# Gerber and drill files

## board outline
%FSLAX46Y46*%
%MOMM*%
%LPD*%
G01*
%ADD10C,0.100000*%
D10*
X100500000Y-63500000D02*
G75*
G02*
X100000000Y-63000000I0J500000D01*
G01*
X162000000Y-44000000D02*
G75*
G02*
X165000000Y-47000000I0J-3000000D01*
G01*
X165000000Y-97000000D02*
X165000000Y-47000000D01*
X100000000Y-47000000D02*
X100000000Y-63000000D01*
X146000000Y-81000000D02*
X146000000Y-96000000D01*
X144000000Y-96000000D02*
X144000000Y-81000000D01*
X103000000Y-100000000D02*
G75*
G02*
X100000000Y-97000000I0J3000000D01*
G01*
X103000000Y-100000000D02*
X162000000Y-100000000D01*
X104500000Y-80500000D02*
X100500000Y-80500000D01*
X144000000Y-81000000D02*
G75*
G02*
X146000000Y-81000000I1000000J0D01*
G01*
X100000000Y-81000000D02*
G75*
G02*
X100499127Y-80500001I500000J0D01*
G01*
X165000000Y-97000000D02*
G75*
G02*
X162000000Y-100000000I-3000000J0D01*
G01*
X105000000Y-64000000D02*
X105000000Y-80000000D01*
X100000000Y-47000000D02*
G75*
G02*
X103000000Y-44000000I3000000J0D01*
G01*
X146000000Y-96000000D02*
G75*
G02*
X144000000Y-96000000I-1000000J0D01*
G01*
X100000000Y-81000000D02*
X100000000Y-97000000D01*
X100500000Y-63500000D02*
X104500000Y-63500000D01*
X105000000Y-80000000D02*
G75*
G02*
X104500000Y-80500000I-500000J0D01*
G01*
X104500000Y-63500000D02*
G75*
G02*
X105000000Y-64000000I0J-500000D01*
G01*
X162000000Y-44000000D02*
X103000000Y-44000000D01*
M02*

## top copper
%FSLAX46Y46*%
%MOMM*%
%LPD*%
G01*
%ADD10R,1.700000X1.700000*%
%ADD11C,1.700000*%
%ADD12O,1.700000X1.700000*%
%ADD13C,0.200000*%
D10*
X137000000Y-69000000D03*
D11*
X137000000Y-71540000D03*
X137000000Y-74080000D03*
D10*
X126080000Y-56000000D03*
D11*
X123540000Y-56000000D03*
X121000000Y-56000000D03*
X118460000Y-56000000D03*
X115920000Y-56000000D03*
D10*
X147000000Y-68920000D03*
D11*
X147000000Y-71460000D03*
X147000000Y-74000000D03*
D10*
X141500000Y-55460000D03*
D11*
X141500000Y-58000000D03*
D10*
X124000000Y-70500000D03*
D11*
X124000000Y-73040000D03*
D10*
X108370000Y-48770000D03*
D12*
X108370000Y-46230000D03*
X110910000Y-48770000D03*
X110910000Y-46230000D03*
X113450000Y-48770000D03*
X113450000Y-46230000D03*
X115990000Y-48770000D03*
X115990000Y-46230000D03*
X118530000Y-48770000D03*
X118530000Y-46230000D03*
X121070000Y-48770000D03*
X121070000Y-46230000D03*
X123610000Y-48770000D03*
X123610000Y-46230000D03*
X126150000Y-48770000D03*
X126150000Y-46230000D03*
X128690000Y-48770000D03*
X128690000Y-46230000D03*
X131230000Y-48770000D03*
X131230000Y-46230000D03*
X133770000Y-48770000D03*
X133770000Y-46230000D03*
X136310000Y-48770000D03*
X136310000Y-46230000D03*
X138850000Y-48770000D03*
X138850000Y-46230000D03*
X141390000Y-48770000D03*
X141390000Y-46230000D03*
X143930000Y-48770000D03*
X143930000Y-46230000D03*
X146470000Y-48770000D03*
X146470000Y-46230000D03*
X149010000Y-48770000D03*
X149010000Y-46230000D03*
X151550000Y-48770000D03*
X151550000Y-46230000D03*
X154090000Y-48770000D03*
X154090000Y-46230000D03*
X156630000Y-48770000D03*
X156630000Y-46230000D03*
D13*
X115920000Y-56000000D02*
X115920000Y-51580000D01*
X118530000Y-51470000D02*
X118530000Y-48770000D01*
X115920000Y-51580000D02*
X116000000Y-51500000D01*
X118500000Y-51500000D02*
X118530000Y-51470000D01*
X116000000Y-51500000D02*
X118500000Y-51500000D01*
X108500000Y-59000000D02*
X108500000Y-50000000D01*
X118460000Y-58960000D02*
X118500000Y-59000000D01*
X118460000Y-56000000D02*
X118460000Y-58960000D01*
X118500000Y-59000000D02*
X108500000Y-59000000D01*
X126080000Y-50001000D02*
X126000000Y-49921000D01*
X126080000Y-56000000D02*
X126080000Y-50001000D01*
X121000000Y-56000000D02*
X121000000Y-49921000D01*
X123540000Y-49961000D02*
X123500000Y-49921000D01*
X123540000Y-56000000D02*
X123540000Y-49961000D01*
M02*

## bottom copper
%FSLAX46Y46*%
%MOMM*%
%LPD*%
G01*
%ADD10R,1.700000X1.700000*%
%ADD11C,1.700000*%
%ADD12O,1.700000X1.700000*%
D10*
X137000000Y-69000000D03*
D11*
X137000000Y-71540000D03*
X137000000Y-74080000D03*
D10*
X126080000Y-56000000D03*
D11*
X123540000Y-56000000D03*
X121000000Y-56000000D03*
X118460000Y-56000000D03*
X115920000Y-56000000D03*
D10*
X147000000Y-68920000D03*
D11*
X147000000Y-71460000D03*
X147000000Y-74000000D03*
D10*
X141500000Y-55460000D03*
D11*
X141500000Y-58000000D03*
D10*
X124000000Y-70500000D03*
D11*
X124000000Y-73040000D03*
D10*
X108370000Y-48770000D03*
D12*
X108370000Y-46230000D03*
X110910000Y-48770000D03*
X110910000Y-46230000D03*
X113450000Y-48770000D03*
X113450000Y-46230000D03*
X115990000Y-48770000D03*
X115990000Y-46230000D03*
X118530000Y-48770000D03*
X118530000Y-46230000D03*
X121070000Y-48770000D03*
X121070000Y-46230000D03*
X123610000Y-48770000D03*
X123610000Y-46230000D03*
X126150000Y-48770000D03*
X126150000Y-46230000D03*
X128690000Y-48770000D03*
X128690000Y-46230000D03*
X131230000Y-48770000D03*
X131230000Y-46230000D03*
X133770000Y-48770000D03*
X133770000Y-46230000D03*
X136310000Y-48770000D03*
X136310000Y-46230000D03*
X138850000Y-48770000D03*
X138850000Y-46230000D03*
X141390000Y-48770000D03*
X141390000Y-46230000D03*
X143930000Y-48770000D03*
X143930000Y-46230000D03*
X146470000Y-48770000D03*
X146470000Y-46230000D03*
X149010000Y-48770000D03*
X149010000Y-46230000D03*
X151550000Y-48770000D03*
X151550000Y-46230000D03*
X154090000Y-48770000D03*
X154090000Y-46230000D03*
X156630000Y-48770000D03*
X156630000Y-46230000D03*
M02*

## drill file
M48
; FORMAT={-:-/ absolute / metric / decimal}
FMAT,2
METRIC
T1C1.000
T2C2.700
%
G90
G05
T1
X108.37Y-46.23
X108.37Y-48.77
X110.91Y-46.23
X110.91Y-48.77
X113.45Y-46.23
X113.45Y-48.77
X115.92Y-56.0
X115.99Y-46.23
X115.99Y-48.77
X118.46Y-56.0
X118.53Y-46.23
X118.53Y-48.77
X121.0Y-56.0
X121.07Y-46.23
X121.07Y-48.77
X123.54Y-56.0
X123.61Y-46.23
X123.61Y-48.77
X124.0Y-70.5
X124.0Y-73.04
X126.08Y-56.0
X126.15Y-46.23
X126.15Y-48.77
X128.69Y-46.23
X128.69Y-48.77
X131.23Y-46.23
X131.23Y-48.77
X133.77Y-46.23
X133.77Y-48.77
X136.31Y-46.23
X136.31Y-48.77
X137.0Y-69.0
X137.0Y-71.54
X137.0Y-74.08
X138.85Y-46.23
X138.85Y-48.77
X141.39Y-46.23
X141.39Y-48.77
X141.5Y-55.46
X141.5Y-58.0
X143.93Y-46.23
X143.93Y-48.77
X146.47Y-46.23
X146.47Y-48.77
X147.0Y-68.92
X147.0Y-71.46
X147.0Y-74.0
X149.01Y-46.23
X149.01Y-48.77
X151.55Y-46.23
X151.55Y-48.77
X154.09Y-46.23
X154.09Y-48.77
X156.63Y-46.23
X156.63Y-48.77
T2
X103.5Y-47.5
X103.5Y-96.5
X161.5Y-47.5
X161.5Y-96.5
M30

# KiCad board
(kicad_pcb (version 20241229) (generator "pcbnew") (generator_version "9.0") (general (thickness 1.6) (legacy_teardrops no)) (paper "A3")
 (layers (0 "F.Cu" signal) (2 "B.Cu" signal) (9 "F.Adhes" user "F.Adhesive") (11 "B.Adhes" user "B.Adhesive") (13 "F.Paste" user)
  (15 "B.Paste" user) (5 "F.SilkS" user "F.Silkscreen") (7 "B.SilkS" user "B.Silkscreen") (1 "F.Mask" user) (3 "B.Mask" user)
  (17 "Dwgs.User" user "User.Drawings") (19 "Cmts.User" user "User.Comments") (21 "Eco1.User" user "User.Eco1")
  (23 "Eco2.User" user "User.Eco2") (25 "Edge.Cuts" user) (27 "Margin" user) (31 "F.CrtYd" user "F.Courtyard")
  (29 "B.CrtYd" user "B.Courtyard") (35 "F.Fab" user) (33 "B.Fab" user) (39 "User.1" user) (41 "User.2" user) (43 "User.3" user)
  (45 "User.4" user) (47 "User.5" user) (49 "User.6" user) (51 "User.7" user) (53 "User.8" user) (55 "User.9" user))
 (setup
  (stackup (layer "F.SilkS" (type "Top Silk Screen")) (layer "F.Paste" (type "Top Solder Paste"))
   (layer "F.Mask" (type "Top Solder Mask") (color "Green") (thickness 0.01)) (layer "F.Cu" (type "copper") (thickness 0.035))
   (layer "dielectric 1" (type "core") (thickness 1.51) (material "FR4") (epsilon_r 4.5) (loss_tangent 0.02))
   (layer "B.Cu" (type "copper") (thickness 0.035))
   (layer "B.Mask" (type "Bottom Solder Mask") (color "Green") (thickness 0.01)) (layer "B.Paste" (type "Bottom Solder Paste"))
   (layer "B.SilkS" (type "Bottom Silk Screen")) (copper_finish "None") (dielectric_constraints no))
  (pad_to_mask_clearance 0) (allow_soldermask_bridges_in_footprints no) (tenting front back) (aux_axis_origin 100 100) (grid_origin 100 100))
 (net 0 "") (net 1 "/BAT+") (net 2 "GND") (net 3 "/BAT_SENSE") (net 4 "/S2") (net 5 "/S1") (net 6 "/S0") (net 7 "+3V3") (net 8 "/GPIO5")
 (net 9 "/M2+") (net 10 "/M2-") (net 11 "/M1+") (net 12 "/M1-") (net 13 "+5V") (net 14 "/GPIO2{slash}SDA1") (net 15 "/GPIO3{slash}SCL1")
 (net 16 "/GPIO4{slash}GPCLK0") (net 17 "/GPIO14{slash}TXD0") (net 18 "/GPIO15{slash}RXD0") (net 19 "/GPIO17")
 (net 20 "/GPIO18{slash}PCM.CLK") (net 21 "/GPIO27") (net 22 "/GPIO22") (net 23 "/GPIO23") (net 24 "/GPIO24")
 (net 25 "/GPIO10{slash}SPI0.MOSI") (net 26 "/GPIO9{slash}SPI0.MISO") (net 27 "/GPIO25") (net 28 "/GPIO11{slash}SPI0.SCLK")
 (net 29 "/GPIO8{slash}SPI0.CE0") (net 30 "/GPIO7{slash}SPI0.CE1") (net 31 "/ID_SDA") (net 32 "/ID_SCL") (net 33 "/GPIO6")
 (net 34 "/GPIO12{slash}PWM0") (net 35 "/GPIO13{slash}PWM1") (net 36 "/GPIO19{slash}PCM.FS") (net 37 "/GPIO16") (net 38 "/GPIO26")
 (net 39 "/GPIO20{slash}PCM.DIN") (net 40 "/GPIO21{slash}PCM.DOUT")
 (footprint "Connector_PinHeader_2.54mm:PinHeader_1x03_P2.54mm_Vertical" (layer "F.Cu") (at 137 69)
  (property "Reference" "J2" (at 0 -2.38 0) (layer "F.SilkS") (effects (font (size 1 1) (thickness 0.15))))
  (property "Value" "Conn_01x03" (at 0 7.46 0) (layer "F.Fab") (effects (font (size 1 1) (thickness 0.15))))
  (pad "1" thru_hole rect (at 0 0) (size 1.7 1.7) (drill 1) (layers "*.Cu" "*.Mask") (remove_unused_layers no) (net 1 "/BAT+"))
  (pad "2" thru_hole circle (at 0 2.54) (size 1.7 1.7) (drill 1) (layers "*.Cu" "*.Mask") (remove_unused_layers no) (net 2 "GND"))
  (pad "3" thru_hole circle (at 0 5.08) (size 1.7 1.7) (drill 1) (layers "*.Cu" "*.Mask") (remove_unused_layers no) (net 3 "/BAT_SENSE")))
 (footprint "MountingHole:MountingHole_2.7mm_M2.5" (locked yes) (layer "F.Cu") (at 161.5 47.5)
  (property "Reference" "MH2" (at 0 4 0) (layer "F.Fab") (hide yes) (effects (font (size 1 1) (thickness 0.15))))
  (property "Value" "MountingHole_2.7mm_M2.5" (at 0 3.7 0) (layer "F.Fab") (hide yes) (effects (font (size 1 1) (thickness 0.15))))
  (pad "" np_thru_hole circle (at 0 0) (size 2.7 2.7) (drill 2.7) (layers "*.Cu" "*.Mask")))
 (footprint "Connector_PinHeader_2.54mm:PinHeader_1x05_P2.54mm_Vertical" (layer "F.Cu") (at 126.08 56 -90)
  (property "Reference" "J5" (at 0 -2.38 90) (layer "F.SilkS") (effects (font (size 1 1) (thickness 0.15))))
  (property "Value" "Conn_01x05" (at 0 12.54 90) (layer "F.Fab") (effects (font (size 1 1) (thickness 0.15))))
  (pad "1" thru_hole rect (at 0 0 270) (size 1.7 1.7) (drill 1) (layers "*.Cu" "*.Mask") (remove_unused_layers no) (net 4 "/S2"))
  (pad "2" thru_hole circle (at 0 2.54 270) (size 1.7 1.7) (drill 1) (layers "*.Cu" "*.Mask") (remove_unused_layers no) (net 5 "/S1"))
  (pad "3" thru_hole circle (at 0 5.08 270) (size 1.7 1.7) (drill 1) (layers "*.Cu" "*.Mask") (remove_unused_layers no) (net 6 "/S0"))
  (pad "4" thru_hole circle (at 0 7.62 270) (size 1.7 1.7) (drill 1) (layers "*.Cu" "*.Mask") (remove_unused_layers no) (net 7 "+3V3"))
  (pad "5" thru_hole circle (at 0 10.16 270) (size 1.7 1.7) (drill 1) (layers "*.Cu" "*.Mask") (remove_unused_layers no) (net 2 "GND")))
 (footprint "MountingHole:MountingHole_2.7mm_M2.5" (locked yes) (layer "F.Cu") (at 103.5 96.5)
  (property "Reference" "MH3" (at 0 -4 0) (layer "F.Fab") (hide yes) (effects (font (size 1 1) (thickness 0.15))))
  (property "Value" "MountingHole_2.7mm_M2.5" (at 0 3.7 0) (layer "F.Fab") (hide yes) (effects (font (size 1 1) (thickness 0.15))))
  (pad "" np_thru_hole circle (at 0 0) (size 2.7 2.7) (drill 2.7) (layers "*.Cu" "*.Mask")))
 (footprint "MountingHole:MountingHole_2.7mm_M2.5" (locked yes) (layer "F.Cu") (at 103.5 47.5)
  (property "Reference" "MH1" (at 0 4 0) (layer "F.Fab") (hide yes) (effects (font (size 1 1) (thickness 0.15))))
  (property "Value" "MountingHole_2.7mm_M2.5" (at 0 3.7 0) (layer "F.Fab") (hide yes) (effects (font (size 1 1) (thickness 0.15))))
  (pad "" np_thru_hole circle (at 0 0) (size 2.7 2.7) (drill 2.7) (layers "*.Cu" "*.Mask")))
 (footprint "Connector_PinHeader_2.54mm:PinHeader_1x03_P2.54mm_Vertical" (layer "F.Cu") (at 147 68.92)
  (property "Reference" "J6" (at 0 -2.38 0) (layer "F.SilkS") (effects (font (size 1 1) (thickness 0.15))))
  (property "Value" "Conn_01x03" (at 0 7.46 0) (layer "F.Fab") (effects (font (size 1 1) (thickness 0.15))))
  (pad "1" thru_hole rect (at 0 0) (size 1.7 1.7) (drill 1) (layers "*.Cu" "*.Mask") (remove_unused_layers no) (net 7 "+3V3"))
  (pad "2" thru_hole circle (at 0 2.54) (size 1.7 1.7) (drill 1) (layers "*.Cu" "*.Mask") (remove_unused_layers no) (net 2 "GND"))
  (pad "3" thru_hole circle (at 0 5.08) (size 1.7 1.7) (drill 1) (layers "*.Cu" "*.Mask") (remove_unused_layers no) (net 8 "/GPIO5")))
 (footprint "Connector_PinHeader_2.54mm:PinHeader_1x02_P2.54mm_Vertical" (layer "F.Cu") (at 141.5 55.46)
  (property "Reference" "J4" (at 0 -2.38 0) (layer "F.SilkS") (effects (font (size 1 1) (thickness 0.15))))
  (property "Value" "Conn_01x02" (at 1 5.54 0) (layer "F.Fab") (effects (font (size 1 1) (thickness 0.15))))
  (pad "1" thru_hole rect (at 0 0) (size 1.7 1.7) (drill 1) (layers "*.Cu" "*.Mask") (remove_unused_layers no) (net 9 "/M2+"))
  (pad "2" thru_hole circle (at 0 2.54) (size 1.7 1.7) (drill 1) (layers "*.Cu" "*.Mask") (remove_unused_layers no) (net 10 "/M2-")))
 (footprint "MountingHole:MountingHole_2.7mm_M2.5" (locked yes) (layer "F.Cu") (at 161.5 96.5)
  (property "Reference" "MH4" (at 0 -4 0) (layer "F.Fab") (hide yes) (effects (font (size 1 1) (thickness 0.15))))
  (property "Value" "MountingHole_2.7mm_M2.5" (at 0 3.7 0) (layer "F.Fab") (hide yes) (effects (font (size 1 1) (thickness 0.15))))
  (pad "" np_thru_hole circle (at 0 0) (size 2.7 2.7) (drill 2.7) (layers "*.Cu" "*.Mask")))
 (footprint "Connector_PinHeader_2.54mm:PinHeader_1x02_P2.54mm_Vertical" (layer "F.Cu") (at 124 70.5)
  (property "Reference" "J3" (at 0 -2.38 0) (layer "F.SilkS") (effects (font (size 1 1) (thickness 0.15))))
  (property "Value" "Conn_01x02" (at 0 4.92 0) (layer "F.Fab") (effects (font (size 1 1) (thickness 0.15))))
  (pad "1" thru_hole rect (at 0 0) (size 1.7 1.7) (drill 1) (layers "*.Cu" "*.Mask") (remove_unused_layers no) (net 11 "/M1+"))
  (pad "2" thru_hole circle (at 0 2.54) (size 1.7 1.7) (drill 1) (layers "*.Cu" "*.Mask") (remove_unused_layers no) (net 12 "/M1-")))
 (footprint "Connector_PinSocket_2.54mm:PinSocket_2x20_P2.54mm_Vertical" (layer "B.Cu") (at 108.37 48.77 -90)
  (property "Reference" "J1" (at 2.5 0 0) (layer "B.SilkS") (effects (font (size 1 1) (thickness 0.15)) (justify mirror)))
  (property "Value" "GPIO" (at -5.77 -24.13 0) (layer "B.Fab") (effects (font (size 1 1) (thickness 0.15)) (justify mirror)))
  (pad "1" thru_hole rect (at 0 0 270) (size 1.7 1.7) (drill 1) (layers "*.Cu" "*.Mask") (remove_unused_layers no) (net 7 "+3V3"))
  (pad "2" thru_hole oval (at -2.54 0 270) (size 1.7 1.7) (drill 1) (layers "*.Cu" "*.Mask") (remove_unused_layers no) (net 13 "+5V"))
  (pad "3" thru_hole oval (at 0 -2.54 270) (size 1.7 1.7) (drill 1) (layers "*.Cu" "*.Mask") (remove_unused_layers no)
   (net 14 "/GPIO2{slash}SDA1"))
  (pad "4" thru_hole oval (at -2.54 -2.54 270) (size 1.7 1.7) (drill 1) (layers "*.Cu" "*.Mask") (remove_unused_layers no) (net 13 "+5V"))
  (pad "5" thru_hole oval (at 0 -5.08 270) (size 1.7 1.7) (drill 1) (layers "*.Cu" "*.Mask") (remove_unused_layers no)
   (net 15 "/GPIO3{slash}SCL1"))
  (pad "6" thru_hole oval (at -2.54 -5.08 270) (size 1.7 1.7) (drill 1) (layers "*.Cu" "*.Mask") (remove_unused_layers no) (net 2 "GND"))
  (pad "7" thru_hole oval (at 0 -7.62 270) (size 1.7 1.7) (drill 1) (layers "*.Cu" "*.Mask") (remove_unused_layers no)
   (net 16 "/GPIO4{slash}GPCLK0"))
  (pad "8" thru_hole oval (at -2.54 -7.62 270) (size 1.7 1.7) (drill 1) (layers "*.Cu" "*.Mask") (remove_unused_layers no)
   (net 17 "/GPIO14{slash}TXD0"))
  (pad "9" thru_hole oval (at 0 -10.16 270) (size 1.7 1.7) (drill 1) (layers "*.Cu" "*.Mask") (remove_unused_layers no) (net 2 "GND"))
  (pad "10" thru_hole oval (at -2.54 -10.16 270) (size 1.7 1.7) (drill 1) (layers "*.Cu" "*.Mask") (remove_unused_layers no)
   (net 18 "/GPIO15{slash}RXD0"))
  (pad "11" thru_hole oval (at 0 -12.7 270) (size 1.7 1.7) (drill 1) (layers "*.Cu" "*.Mask") (remove_unused_layers no) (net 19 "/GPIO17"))
  (pad "12" thru_hole oval (at -2.54 -12.7 270) (size 1.7 1.7) (drill 1) (layers "*.Cu" "*.Mask") (remove_unused_layers no)
   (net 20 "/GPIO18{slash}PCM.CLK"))
  (pad "13" thru_hole oval (at 0 -15.24 270) (size 1.7 1.7) (drill 1) (layers "*.Cu" "*.Mask") (remove_unused_layers no) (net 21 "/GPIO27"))
  (pad "14" thru_hole oval (at -2.54 -15.24 270) (size 1.7 1.7) (drill 1) (layers "*.Cu" "*.Mask") (remove_unused_layers no) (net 2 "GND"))
  (pad "15" thru_hole oval (at 0 -17.78 270) (size 1.7 1.7) (drill 1) (layers "*.Cu" "*.Mask") (remove_unused_layers no) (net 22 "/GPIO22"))
  (pad "16" thru_hole oval (at -2.54 -17.78 270) (size 1.7 1.7) (drill 1) (layers "*.Cu" "*.Mask") (remove_unused_layers no)
   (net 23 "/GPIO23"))
  (pad "17" thru_hole oval (at 0 -20.32 270) (size 1.7 1.7) (drill 1) (layers "*.Cu" "*.Mask") (remove_unused_layers no) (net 7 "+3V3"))
  (pad "18" thru_hole oval (at -2.54 -20.32 270) (size 1.7 1.7) (drill 1) (layers "*.Cu" "*.Mask") (remove_unused_layers no)
   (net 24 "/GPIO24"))
  (pad "19" thru_hole oval (at 0 -22.86 270) (size 1.7 1.7) (drill 1) (layers "*.Cu" "*.Mask") (remove_unused_layers no)
   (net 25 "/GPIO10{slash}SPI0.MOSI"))
  (pad "20" thru_hole oval (at -2.54 -22.86 270) (size 1.7 1.7) (drill 1) (layers "*.Cu" "*.Mask") (remove_unused_layers no) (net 2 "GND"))
  (pad "21" thru_hole oval (at 0 -25.4 270) (size 1.7 1.7) (drill 1) (layers "*.Cu" "*.Mask") (remove_unused_layers no)
   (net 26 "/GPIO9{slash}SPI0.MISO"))
  (pad "22" thru_hole oval (at -2.54 -25.4 270) (size 1.7 1.7) (drill 1) (layers "*.Cu" "*.Mask") (remove_unused_layers no)
   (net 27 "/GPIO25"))
  (pad "23" thru_hole oval (at 0 -27.94 270) (size 1.7 1.7) (drill 1) (layers "*.Cu" "*.Mask") (remove_unused_layers no)
   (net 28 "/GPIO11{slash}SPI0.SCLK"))
  (pad "24" thru_hole oval (at -2.54 -27.94 270) (size 1.7 1.7) (drill 1) (layers "*.Cu" "*.Mask") (remove_unused_layers no)
   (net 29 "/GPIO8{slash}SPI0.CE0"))
  (pad "25" thru_hole oval (at 0 -30.48 270) (size 1.7 1.7) (drill 1) (layers "*.Cu" "*.Mask") (remove_unused_layers no) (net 2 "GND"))
  (pad "26" thru_hole oval (at -2.54 -30.48 270) (size 1.7 1.7) (drill 1) (layers "*.Cu" "*.Mask") (remove_unused_layers no)
   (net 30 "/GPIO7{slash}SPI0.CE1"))
  (pad "27" thru_hole oval (at 0 -33.02 270) (size 1.7 1.7) (drill 1) (layers "*.Cu" "*.Mask") (remove_unused_layers no) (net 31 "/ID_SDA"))
  (pad "28" thru_hole oval (at -2.54 -33.02 270) (size 1.7 1.7) (drill 1) (layers "*.Cu" "*.Mask") (remove_unused_layers no)
   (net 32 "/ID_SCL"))
  (pad "29" thru_hole oval (at 0 -35.56 270) (size 1.7 1.7) (drill 1) (layers "*.Cu" "*.Mask") (remove_unused_layers no) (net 8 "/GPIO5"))
  (pad "30" thru_hole oval (at -2.54 -35.56 270) (size 1.7 1.7) (drill 1) (layers "*.Cu" "*.Mask") (remove_unused_layers no) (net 2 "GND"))
  (pad "31" thru_hole oval (at 0 -38.1 270) (size 1.7 1.7) (drill 1) (layers "*.Cu" "*.Mask") (remove_unused_layers no) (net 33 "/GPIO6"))
  (pad "32" thru_hole oval (at -2.54 -38.1 270) (size 1.7 1.7) (drill 1) (layers "*.Cu" "*.Mask") (remove_unused_layers no)
   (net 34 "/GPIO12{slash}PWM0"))
  (pad "33" thru_hole oval (at 0 -40.64 270) (size 1.7 1.7) (drill 1) (layers "*.Cu" "*.Mask") (remove_unused_layers no)
   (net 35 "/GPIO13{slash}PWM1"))
  (pad "34" thru_hole oval (at -2.54 -40.64 270) (size 1.7 1.7) (drill 1) (layers "*.Cu" "*.Mask") (remove_unused_layers no) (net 2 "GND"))
  (pad "35" thru_hole oval (at 0 -43.18 270) (size 1.7 1.7) (drill 1) (layers "*.Cu" "*.Mask") (remove_unused_layers no)
   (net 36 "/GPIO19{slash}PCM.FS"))
  (pad "36" thru_hole oval (at -2.54 -43.18 270) (size 1.7 1.7) (drill 1) (layers "*.Cu" "*.Mask") (remove_unused_layers no)
   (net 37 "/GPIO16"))
  (pad "37" thru_hole oval (at 0 -45.72 270) (size 1.7 1.7) (drill 1) (layers "*.Cu" "*.Mask") (remove_unused_layers no) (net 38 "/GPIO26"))
  (pad "38" thru_hole oval (at -2.54 -45.72 270) (size 1.7 1.7) (drill 1) (layers "*.Cu" "*.Mask") (remove_unused_layers no)
   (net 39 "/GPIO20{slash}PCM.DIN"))
  (pad "39" thru_hole oval (at 0 -48.26 270) (size 1.7 1.7) (drill 1) (layers "*.Cu" "*.Mask") (remove_unused_layers no) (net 2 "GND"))
  (pad "40" thru_hole oval (at -2.54 -48.26 270) (size 1.7 1.7) (drill 1) (layers "*.Cu" "*.Mask") (remove_unused_layers no)
   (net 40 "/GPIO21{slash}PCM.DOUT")))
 (gr_arc (start 100.5 63.5) (mid 100.146447 63.353553) (end 100 63) (stroke (width 0.1) (type solid)) (layer "Edge.Cuts"))
 (gr_arc (start 162 44) (mid 164.12132 44.87868) (end 165 47) (stroke (width 0.1) (type solid)) (layer "Edge.Cuts"))
 (gr_line (start 165 97) (end 165 47) (stroke (width 0.1) (type solid)) (layer "Edge.Cuts"))
 (gr_line (start 100 47) (end 100 63) (stroke (width 0.1) (type solid)) (layer "Edge.Cuts"))
 (gr_line (start 146 81) (end 146 96) (stroke (width 0.1) (type solid)) (layer "Edge.Cuts"))
 (gr_line (start 144 96) (end 144 81) (stroke (width 0.1) (type solid)) (layer "Edge.Cuts"))
 (gr_arc (start 103 100) (mid 100.87868 99.12132) (end 100 97) (stroke (width 0.1) (type solid)) (layer "Edge.Cuts"))
 (gr_line (start 103 100) (end 162 100) (stroke (width 0.1) (type solid)) (layer "Edge.Cuts"))
 (gr_line (start 104.5 80.5) (end 100.5 80.5) (stroke (width 0.1) (type solid)) (layer "Edge.Cuts"))
 (gr_arc (start 144 81) (mid 145 80) (end 146 81) (stroke (width 0.1) (type solid)) (layer "Edge.Cuts"))
 (gr_arc (start 100 81) (mid 100.146138 80.646755) (end 100.499127 80.500001) (stroke (width 0.1) (type solid)) (layer "Edge.Cuts"))
 (gr_arc (start 165 97) (mid 164.12132 99.12132) (end 162 100) (stroke (width 0.1) (type solid)) (layer "Edge.Cuts"))
 (gr_line (start 105 64) (end 105 80) (stroke (width 0.1) (type solid)) (layer "Edge.Cuts"))
 (gr_arc (start 100 47) (mid 100.87868 44.87868) (end 103 44) (stroke (width 0.1) (type solid)) (layer "Edge.Cuts"))
 (gr_arc (start 146 96) (mid 145 97) (end 144 96) (stroke (width 0.1) (type solid)) (layer "Edge.Cuts"))
 (gr_line (start 100 81) (end 100 97) (stroke (width 0.1) (type solid)) (layer "Edge.Cuts"))
 (gr_line (start 100.5 63.5) (end 104.5 63.5) (stroke (width 0.1) (type solid)) (layer "Edge.Cuts"))
 (gr_arc (start 105 80) (mid 104.853553 80.353553) (end 104.5 80.5) (stroke (width 0.1) (type solid)) (layer "Edge.Cuts"))
 (gr_arc (start 104.5 63.5) (mid 104.853553 63.646447) (end 105 64) (stroke (width 0.1) (type solid)) (layer "Edge.Cuts"))
 (gr_line (start 162 44) (end 103 44) (stroke (width 0.1) (type solid)) (layer "Edge.Cuts"))
 (segment (start 115.92 56) (end 115.92 51.58) (width 0.2) (layer "F.Cu") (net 2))
 (segment (start 118.53 51.47) (end 118.53 48.77) (width 0.2) (layer "F.Cu") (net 2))
 (segment (start 115.92 51.58) (end 116 51.5) (width 0.2) (layer "F.Cu") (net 2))
 (segment (start 118.5 51.5) (end 118.53 51.47) (width 0.2) (layer "F.Cu") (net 2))
 (segment (start 116 51.5) (end 118.5 51.5) (width 0.2) (layer "F.Cu") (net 2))
 (segment (start 108.5 59) (end 108.5 50) (width 0.2) (layer "F.Cu") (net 7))
 (segment (start 118.46 58.96) (end 118.5 59) (width 0.2) (layer "F.Cu") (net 7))
 (segment (start 118.46 56) (end 118.46 58.96) (width 0.2) (layer "F.Cu") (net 7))
 (segment (start 118.5 59) (end 108.5 59) (width 0.2) (layer "F.Cu") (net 7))
 (segment (start 126.08 50.001) (end 126 49.921) (width 0.2) (layer "F.Cu") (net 4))
 (segment (start 126.08 56) (end 126.08 50.001) (width 0.2) (layer "F.Cu") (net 4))
 (segment (start 121 56) (end 121 49.921) (width 0.2) (layer "F.Cu") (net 6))
 (segment (start 123.54 49.961) (end 123.5 49.921) (width 0.2) (layer "F.Cu") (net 5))
 (segment (start 123.54 56) (end 123.54 49.961) (width 0.2) (layer "F.Cu") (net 5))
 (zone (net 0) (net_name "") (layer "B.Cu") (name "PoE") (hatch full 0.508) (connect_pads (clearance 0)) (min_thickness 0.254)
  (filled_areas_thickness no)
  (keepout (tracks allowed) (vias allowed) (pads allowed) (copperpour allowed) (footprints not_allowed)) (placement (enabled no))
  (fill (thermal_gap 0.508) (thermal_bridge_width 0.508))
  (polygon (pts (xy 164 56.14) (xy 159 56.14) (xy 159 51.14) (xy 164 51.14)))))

